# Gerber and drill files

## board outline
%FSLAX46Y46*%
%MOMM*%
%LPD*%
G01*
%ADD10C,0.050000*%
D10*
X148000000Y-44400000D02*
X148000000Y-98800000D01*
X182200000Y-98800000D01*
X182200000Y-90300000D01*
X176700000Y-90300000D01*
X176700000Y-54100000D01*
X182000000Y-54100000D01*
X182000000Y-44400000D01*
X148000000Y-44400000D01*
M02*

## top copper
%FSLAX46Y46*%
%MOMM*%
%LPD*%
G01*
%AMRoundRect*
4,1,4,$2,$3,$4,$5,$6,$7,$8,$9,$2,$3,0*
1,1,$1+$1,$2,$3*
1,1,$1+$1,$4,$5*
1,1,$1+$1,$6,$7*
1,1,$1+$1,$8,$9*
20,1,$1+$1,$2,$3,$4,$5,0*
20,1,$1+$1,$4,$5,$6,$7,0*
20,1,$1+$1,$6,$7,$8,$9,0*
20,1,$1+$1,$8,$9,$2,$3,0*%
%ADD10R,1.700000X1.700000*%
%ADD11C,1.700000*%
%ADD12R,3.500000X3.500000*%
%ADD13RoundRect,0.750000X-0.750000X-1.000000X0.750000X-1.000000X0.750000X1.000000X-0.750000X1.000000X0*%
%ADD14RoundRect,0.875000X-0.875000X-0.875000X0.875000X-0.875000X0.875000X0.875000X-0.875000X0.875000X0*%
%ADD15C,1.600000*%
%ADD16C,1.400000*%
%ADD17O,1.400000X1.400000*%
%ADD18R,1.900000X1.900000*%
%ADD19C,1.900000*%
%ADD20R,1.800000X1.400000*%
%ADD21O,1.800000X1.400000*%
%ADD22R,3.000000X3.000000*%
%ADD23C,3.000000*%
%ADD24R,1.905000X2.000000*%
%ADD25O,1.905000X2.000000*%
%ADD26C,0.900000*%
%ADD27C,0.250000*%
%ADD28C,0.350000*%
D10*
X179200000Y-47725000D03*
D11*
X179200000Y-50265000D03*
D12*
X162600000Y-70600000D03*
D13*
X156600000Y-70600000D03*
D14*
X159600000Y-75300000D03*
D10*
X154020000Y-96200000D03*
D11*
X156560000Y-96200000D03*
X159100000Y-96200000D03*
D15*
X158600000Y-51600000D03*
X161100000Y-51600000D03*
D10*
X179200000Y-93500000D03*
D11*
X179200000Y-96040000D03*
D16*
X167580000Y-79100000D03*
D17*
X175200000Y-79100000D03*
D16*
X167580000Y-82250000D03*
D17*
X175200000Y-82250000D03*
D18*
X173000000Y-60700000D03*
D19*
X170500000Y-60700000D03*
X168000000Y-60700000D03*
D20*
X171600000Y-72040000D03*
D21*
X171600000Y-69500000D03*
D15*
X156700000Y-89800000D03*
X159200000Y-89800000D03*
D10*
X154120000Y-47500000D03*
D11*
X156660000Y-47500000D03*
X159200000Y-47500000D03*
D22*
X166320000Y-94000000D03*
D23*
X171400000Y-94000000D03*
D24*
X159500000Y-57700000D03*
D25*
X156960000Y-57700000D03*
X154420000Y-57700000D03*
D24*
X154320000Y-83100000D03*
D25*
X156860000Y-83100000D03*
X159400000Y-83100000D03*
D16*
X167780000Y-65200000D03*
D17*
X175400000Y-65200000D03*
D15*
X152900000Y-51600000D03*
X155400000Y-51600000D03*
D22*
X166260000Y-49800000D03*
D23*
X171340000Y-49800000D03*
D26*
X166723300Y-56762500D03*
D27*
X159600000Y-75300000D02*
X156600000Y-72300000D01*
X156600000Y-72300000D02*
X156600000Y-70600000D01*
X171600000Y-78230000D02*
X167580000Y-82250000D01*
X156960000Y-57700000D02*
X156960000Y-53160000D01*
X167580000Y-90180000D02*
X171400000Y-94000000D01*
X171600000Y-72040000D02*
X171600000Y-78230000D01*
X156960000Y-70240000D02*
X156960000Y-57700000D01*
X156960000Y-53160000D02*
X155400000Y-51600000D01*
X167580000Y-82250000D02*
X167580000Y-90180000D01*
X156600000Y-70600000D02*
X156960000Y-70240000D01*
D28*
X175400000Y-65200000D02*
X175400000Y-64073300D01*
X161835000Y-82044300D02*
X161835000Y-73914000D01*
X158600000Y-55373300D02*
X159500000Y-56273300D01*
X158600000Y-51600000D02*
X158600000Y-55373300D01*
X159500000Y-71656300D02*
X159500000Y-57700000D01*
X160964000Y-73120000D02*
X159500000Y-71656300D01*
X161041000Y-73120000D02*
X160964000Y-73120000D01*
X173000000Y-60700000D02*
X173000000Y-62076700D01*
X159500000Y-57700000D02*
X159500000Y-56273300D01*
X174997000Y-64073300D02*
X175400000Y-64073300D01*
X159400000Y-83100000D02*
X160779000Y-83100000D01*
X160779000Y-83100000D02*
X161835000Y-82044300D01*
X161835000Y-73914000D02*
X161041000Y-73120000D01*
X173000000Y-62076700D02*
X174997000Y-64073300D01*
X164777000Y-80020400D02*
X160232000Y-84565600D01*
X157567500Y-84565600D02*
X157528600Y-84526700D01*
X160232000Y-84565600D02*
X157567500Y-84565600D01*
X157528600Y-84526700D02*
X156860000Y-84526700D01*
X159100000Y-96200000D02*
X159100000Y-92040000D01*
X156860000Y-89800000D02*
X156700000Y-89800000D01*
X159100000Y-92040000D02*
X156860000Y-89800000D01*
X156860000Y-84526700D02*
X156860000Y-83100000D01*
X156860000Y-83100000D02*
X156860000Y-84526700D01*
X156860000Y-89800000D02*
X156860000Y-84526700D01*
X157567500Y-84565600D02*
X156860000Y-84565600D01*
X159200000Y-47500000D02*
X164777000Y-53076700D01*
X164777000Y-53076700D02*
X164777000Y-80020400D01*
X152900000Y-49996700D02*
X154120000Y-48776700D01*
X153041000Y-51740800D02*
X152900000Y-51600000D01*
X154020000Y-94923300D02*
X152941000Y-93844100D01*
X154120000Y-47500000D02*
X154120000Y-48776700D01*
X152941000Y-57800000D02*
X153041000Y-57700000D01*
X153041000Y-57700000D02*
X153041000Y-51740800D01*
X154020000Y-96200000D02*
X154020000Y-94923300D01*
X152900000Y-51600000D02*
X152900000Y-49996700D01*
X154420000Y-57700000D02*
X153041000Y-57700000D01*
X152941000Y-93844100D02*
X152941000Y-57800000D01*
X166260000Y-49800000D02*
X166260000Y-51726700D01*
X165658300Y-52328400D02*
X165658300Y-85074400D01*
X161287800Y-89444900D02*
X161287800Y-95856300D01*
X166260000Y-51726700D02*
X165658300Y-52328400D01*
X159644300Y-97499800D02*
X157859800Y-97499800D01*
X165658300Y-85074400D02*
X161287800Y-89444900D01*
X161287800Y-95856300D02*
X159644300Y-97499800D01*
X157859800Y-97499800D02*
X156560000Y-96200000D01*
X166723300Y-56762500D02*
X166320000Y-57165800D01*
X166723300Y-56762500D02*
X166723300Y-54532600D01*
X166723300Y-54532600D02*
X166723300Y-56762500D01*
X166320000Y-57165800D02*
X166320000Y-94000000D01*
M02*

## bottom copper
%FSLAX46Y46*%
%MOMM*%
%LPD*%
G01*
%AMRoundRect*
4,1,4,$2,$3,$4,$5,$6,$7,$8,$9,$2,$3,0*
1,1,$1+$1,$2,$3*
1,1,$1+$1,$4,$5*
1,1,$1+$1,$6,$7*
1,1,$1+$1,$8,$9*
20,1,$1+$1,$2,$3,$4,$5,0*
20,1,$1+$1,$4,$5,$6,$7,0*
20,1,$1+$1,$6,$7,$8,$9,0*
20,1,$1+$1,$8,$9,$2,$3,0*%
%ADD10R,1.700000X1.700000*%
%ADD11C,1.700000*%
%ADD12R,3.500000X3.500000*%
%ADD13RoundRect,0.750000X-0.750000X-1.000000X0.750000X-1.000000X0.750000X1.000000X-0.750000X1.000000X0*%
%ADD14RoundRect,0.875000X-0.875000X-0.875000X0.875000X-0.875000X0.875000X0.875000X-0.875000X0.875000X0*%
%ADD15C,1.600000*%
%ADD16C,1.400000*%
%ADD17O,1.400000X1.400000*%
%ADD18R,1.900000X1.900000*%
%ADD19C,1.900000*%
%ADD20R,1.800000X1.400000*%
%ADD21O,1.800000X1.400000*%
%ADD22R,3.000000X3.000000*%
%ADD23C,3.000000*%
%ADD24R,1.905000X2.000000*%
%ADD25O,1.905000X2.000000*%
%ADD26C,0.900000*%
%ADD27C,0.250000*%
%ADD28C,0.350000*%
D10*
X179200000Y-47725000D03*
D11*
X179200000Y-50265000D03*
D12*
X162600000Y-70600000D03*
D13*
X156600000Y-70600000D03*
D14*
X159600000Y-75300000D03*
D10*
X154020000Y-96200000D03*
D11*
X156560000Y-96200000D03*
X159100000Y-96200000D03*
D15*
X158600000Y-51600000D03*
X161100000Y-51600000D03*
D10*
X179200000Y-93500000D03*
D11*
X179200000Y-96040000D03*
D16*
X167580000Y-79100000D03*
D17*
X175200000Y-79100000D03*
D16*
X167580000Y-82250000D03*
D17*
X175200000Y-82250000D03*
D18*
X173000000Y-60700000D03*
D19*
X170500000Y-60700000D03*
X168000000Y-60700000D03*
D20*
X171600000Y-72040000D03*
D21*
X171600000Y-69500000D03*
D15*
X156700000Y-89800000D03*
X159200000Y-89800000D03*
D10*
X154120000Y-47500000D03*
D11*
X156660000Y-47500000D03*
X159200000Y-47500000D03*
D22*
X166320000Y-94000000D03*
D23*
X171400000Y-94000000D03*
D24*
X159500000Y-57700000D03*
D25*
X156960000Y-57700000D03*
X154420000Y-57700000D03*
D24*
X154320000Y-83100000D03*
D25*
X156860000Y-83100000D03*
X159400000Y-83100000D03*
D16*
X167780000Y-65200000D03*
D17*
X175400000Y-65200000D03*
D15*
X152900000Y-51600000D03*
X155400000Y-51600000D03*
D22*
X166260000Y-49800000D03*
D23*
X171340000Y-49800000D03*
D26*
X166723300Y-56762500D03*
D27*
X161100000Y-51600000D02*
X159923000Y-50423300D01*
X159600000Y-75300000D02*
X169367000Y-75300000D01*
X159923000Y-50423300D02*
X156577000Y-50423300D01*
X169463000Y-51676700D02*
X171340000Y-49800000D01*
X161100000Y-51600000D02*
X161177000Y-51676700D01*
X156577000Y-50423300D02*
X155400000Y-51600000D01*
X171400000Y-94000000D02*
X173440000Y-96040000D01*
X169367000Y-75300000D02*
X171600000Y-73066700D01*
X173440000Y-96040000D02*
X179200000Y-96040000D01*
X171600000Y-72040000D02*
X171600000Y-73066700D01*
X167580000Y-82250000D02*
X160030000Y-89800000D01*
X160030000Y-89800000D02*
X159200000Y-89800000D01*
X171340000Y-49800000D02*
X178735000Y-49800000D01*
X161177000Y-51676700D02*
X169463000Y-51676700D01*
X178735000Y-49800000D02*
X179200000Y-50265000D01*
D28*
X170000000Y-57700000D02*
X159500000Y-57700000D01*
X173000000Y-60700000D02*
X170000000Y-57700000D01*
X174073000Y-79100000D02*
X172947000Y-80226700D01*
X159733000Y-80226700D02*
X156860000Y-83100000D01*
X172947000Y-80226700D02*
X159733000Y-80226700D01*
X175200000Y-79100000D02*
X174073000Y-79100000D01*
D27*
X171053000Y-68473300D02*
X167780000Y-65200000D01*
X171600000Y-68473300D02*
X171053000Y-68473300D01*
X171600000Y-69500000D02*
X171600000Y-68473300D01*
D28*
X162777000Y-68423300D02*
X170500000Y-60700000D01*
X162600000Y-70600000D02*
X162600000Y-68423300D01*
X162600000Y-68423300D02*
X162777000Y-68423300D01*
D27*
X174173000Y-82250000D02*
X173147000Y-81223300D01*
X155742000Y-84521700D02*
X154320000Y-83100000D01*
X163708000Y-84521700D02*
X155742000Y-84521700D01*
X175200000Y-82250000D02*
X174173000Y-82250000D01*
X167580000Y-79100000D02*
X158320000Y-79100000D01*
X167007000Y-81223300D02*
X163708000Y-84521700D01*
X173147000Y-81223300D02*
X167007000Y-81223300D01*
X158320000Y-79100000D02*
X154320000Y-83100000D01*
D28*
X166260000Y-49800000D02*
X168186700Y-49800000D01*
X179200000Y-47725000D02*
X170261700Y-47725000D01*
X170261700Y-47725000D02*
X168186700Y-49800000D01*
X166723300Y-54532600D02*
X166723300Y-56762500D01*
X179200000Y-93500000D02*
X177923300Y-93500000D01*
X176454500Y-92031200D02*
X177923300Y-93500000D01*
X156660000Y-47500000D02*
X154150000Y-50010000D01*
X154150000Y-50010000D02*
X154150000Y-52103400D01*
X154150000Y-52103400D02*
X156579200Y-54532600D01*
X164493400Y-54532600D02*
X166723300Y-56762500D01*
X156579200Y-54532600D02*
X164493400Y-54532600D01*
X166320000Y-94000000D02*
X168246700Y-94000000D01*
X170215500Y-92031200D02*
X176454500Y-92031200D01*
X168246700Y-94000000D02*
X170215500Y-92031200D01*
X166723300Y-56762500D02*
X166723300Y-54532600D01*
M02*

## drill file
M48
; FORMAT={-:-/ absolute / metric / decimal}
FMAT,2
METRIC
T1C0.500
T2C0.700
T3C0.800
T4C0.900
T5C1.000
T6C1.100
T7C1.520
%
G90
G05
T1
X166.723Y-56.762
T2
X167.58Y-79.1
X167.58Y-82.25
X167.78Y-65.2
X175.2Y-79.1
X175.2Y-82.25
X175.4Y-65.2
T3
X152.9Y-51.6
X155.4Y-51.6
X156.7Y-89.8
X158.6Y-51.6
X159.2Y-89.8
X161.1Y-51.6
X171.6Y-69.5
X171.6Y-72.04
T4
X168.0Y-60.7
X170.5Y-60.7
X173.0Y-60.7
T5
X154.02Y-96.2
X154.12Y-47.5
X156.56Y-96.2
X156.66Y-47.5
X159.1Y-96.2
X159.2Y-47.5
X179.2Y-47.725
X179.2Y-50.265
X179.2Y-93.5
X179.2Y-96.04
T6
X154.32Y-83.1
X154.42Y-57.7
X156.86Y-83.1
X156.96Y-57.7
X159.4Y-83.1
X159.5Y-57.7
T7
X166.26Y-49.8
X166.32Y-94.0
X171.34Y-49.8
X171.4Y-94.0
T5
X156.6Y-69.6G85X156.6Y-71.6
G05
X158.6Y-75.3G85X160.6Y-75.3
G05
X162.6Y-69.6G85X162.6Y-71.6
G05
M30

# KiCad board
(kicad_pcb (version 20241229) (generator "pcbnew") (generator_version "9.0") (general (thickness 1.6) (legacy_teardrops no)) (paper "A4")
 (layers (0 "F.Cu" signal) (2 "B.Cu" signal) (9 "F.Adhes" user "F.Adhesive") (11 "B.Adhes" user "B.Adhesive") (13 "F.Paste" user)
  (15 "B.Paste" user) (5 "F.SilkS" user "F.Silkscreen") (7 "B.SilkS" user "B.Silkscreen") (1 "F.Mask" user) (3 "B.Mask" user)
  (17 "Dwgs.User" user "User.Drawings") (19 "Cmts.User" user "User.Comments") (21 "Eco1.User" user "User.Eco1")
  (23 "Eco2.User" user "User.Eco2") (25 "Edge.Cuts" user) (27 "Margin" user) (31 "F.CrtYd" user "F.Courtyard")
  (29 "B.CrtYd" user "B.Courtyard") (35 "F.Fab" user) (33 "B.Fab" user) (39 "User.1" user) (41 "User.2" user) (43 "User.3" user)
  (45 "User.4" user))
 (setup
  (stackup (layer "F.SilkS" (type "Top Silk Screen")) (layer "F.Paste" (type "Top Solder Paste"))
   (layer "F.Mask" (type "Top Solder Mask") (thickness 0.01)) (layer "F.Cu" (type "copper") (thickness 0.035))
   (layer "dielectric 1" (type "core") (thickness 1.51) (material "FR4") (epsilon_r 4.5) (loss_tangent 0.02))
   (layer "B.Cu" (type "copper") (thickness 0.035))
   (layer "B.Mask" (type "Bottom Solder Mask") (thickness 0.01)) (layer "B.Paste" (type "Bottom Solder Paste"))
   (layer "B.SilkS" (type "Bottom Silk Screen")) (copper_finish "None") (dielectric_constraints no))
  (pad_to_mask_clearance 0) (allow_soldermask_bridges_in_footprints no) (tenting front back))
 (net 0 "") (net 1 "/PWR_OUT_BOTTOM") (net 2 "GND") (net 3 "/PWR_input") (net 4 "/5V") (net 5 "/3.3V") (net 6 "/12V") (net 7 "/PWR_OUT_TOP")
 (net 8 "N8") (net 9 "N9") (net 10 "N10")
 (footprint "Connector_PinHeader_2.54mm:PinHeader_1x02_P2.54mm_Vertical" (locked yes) (layer "F.Cu") (at 179.2 47.725)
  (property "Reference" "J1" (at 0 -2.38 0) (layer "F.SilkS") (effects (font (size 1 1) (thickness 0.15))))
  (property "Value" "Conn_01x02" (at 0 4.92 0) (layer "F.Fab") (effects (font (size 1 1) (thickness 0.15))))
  (pad "1" thru_hole rect (at 0 0) (size 1.7 1.7) (drill 1) (layers "*.Cu" "*.Mask") (remove_unused_layers no) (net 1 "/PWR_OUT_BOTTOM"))
  (pad "2" thru_hole circle (at 0 2.54) (size 1.7 1.7) (drill 1) (layers "*.Cu" "*.Mask") (remove_unused_layers no) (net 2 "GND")))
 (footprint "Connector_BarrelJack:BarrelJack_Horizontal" (layer "F.Cu") (at 162.6 70.6)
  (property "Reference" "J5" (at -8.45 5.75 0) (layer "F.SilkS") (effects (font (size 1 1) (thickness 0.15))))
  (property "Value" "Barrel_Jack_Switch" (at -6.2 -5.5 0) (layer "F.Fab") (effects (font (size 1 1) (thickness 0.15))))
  (pad "1" thru_hole rect (at 0 0) (size 3.5 3.5) (drill oval 1 3) (layers "*.Cu" "*.Mask") (remove_unused_layers no) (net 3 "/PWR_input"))
  (pad "2" thru_hole roundrect (at -6 0) (size 3 3.5) (drill oval 1 3) (layers "*.Cu" "*.Mask") (remove_unused_layers no)
   (roundrect_rratio 0.25) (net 2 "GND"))
  (pad "3" thru_hole roundrect (at -3 4.7) (size 3.5 3.5) (drill oval 3 1) (layers "*.Cu" "*.Mask") (remove_unused_layers no)
   (roundrect_rratio 0.25) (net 2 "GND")))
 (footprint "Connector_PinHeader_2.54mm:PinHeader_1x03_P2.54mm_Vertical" (layer "F.Cu") (at 154.02 96.2 90)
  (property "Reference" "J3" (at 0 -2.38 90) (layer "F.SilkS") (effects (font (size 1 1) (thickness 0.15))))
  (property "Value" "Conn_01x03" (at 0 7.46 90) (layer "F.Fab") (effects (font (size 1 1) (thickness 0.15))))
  (pad "1" thru_hole rect (at 0 0 90) (size 1.7 1.7) (drill 1) (layers "*.Cu" "*.Mask") (remove_unused_layers no) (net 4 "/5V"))
  (pad "2" thru_hole circle (at 0 2.54 90) (size 1.7 1.7) (drill 1) (layers "*.Cu" "*.Mask") (remove_unused_layers no)
   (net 1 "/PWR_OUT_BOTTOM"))
  (pad "3" thru_hole circle (at 0 5.08 90) (size 1.7 1.7) (drill 1) (layers "*.Cu" "*.Mask") (remove_unused_layers no) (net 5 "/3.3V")))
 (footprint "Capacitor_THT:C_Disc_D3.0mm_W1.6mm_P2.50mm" (layer "F.Cu") (at 158.6 51.6)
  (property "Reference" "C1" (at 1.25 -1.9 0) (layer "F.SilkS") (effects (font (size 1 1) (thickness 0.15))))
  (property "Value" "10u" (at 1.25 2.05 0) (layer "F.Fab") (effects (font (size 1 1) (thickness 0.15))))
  (pad "1" thru_hole circle (at 0 0) (size 1.6 1.6) (drill 0.8) (layers "*.Cu" "*.Mask") (remove_unused_layers no) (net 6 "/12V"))
  (pad "2" thru_hole circle (at 2.5 0) (size 1.6 1.6) (drill 0.8) (layers "*.Cu" "*.Mask") (remove_unused_layers no) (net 2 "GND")))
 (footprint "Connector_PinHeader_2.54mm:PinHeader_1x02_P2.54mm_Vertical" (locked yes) (layer "F.Cu") (at 179.2 93.5)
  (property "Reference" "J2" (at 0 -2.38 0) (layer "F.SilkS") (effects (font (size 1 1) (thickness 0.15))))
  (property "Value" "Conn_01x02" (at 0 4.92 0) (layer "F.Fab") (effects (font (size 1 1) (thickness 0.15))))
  (pad "1" thru_hole rect (at 0 0) (size 1.7 1.7) (drill 1) (layers "*.Cu" "*.Mask") (remove_unused_layers no) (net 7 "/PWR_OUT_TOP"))
  (pad "2" thru_hole circle (at 0 2.54) (size 1.7 1.7) (drill 1) (layers "*.Cu" "*.Mask") (remove_unused_layers no) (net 2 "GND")))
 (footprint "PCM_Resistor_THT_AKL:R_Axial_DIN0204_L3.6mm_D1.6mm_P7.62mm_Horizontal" (layer "F.Cu") (at 167.58 79.1)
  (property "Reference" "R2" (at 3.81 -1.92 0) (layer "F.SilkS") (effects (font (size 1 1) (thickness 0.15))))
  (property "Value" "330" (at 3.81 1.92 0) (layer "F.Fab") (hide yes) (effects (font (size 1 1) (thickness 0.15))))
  (pad "1" thru_hole circle (at 0 0) (size 1.4 1.4) (drill 0.7) (layers "*.Cu" "*.Mask") (remove_unused_layers no) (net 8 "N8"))
  (pad "2" thru_hole oval (at 7.62 0) (size 1.4 1.4) (drill 0.7) (layers "*.Cu" "*.Mask") (remove_unused_layers no) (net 5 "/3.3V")))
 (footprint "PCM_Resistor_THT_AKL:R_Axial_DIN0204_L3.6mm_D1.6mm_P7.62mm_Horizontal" (layer "F.Cu") (at 167.58 82.25)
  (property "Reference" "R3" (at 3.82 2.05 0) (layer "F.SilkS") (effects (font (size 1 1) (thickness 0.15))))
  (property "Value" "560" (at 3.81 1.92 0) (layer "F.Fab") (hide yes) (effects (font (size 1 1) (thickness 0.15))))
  (pad "1" thru_hole circle (at 0 0) (size 1.4 1.4) (drill 0.7) (layers "*.Cu" "*.Mask") (remove_unused_layers no) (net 2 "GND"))
  (pad "2" thru_hole oval (at 7.62 0) (size 1.4 1.4) (drill 0.7) (layers "*.Cu" "*.Mask") (remove_unused_layers no) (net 8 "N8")))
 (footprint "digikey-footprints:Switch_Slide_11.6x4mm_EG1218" (layer "F.Cu") (at 173 60.7 180)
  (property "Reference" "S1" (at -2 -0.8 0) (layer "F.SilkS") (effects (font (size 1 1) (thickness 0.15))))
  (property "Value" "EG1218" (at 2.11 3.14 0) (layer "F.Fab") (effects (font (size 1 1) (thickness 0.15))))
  (pad "1" thru_hole rect (at 0 0 180) (size 1.9 1.9) (drill 0.9) (layers "*.Cu" "*.Mask") (remove_unused_layers no) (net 6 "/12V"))
  (pad "2" thru_hole circle (at 2.5 0 180) (size 1.9 1.9) (drill 0.9) (layers "*.Cu" "*.Mask") (remove_unused_layers no)
   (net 3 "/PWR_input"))
  (pad "3" thru_hole circle (at 5 0 180) (size 1.9 1.9) (drill 0.9) (layers "*.Cu" "*.Mask") (remove_unused_layers no) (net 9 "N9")))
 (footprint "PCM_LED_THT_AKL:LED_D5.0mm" (layer "F.Cu") (at 171.6 72.04 90)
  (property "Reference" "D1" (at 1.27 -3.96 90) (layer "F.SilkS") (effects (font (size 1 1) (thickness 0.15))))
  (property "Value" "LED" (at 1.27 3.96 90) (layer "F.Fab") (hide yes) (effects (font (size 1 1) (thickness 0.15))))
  (pad "1" thru_hole rect (at 0 0 90) (size 1.4 1.8) (drill 0.8) (layers "*.Cu" "*.Mask") (remove_unused_layers no) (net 2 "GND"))
  (pad "2" thru_hole oval (at 2.54 0 90) (size 1.4 1.8) (drill 0.8) (layers "*.Cu" "*.Mask") (remove_unused_layers no) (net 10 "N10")))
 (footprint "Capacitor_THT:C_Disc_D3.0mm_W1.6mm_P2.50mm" (layer "F.Cu") (at 156.7 89.8)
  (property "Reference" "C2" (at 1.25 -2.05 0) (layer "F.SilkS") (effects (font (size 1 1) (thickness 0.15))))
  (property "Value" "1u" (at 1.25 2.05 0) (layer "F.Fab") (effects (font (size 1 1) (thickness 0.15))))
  (pad "1" thru_hole circle (at 0 0) (size 1.6 1.6) (drill 0.8) (layers "*.Cu" "*.Mask") (remove_unused_layers no) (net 5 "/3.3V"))
  (pad "2" thru_hole circle (at 2.5 0) (size 1.6 1.6) (drill 0.8) (layers "*.Cu" "*.Mask") (remove_unused_layers no) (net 2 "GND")))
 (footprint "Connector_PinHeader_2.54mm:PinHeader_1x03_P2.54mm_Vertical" (layer "F.Cu") (at 154.12 47.5 90)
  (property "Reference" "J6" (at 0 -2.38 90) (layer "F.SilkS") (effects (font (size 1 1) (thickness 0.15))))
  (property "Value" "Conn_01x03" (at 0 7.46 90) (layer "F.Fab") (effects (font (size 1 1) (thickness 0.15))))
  (pad "1" thru_hole rect (at 0 0 90) (size 1.7 1.7) (drill 1) (layers "*.Cu" "*.Mask") (remove_unused_layers no) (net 4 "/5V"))
  (pad "2" thru_hole circle (at 0 2.54 90) (size 1.7 1.7) (drill 1) (layers "*.Cu" "*.Mask") (remove_unused_layers no)
   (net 7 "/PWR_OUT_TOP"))
  (pad "3" thru_hole circle (at 0 5.08 90) (size 1.7 1.7) (drill 1) (layers "*.Cu" "*.Mask") (remove_unused_layers no) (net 5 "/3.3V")))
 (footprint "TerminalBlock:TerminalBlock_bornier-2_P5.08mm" (layer "F.Cu") (at 166.32 94)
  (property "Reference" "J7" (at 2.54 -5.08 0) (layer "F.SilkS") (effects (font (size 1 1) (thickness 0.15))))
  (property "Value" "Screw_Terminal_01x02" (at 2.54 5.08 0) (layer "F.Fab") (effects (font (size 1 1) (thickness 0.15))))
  (pad "1" thru_hole rect (at 0 0) (size 3 3) (drill 1.52) (layers "*.Cu" "*.Mask") (remove_unused_layers no) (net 7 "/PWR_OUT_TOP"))
  (pad "2" thru_hole circle (at 5.08 0) (size 3 3) (drill 1.52) (layers "*.Cu" "*.Mask") (remove_unused_layers no) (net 2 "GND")))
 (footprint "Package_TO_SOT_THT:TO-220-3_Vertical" (layer "F.Cu") (at 159.5 57.7 180)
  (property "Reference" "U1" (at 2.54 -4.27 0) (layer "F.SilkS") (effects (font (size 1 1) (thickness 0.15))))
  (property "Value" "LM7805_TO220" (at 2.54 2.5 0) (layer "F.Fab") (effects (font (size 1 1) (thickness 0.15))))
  (pad "1" thru_hole rect (at 0 0 180) (size 1.905 2) (drill 1.1) (layers "*.Cu" "*.Mask") (remove_unused_layers no) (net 6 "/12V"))
  (pad "2" thru_hole oval (at 2.54 0 180) (size 1.905 2) (drill 1.1) (layers "*.Cu" "*.Mask") (remove_unused_layers no) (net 2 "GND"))
  (pad "3" thru_hole oval (at 5.08 0 180) (size 1.905 2) (drill 1.1) (layers "*.Cu" "*.Mask") (remove_unused_layers no) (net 4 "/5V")))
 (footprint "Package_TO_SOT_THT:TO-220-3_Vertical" (layer "F.Cu") (at 154.32 83.1)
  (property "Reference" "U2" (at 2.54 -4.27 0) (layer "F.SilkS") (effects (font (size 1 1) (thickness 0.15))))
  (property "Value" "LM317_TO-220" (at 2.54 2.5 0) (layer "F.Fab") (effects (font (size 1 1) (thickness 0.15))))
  (pad "1" thru_hole rect (at 0 0) (size 1.905 2) (drill 1.1) (layers "*.Cu" "*.Mask") (remove_unused_layers no) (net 8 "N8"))
  (pad "2" thru_hole oval (at 2.54 0) (size 1.905 2) (drill 1.1) (layers "*.Cu" "*.Mask") (remove_unused_layers no) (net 5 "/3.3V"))
  (pad "3" thru_hole oval (at 5.08 0) (size 1.905 2) (drill 1.1) (layers "*.Cu" "*.Mask") (remove_unused_layers no) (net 6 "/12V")))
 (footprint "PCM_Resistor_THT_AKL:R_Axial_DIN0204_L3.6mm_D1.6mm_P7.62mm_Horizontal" (layer "F.Cu") (at 167.78 65.2)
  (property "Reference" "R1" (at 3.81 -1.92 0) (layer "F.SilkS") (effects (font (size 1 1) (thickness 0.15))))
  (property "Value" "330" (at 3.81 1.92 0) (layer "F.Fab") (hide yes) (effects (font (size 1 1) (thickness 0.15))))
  (pad "1" thru_hole circle (at 0 0) (size 1.4 1.4) (drill 0.7) (layers "*.Cu" "*.Mask") (remove_unused_layers no) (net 10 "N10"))
  (pad "2" thru_hole oval (at 7.62 0) (size 1.4 1.4) (drill 0.7) (layers "*.Cu" "*.Mask") (remove_unused_layers no) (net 6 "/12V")))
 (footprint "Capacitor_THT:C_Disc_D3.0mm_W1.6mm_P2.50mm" (layer "F.Cu") (at 152.9 51.6)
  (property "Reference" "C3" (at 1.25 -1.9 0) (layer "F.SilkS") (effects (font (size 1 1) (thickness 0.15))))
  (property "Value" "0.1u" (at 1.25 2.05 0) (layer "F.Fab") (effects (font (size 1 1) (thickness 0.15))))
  (pad "1" thru_hole circle (at 0 0) (size 1.6 1.6) (drill 0.8) (layers "*.Cu" "*.Mask") (remove_unused_layers no) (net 4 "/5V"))
  (pad "2" thru_hole circle (at 2.5 0) (size 1.6 1.6) (drill 0.8) (layers "*.Cu" "*.Mask") (remove_unused_layers no) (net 2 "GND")))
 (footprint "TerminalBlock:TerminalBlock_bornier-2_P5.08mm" (layer "F.Cu") (at 166.26 49.8)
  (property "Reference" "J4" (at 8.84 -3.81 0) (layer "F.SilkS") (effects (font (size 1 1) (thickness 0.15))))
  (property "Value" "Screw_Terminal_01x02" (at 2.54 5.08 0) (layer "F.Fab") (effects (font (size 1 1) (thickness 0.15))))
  (pad "1" thru_hole rect (at 0 0) (size 3 3) (drill 1.52) (layers "*.Cu" "*.Mask") (remove_unused_layers no) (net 1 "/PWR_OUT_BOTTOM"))
  (pad "2" thru_hole circle (at 5.08 0) (size 3 3) (drill 1.52) (layers "*.Cu" "*.Mask") (remove_unused_layers no) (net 2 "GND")))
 (gr_poly
  (pts (xy 148 44.4) (xy 148 98.8) (xy 182.2 98.8) (xy 182.2 90.3) (xy 176.7 90.3) (xy 176.7 54.1) (xy 182 54.1) (xy 182 44.4))
  (stroke (width 0.05) (type solid)) (fill no) (layer "Edge.Cuts"))
 (segment (start 159.6 75.3) (end 156.6 72.3) (width 0.25) (layer "F.Cu") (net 2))
 (segment (start 156.6 72.3) (end 156.6 70.6) (width 0.25) (layer "F.Cu") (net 2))
 (segment (start 171.6 78.23) (end 167.58 82.25) (width 0.25) (layer "F.Cu") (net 2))
 (segment (start 156.96 57.7) (end 156.96 53.16) (width 0.25) (layer "F.Cu") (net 2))
 (segment (start 167.58 90.18) (end 171.4 94) (width 0.25) (layer "F.Cu") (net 2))
 (segment (start 171.6 72.04) (end 171.6 78.23) (width 0.25) (layer "F.Cu") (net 2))
 (segment (start 156.96 70.24) (end 156.96 57.7) (width 0.25) (layer "F.Cu") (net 2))
 (segment (start 156.96 53.16) (end 155.4 51.6) (width 0.25) (layer "F.Cu") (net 2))
 (segment (start 167.58 82.25) (end 167.58 90.18) (width 0.25) (layer "F.Cu") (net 2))
 (segment (start 156.6 70.6) (end 156.96 70.24) (width 0.25) (layer "F.Cu") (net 2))
 (segment (start 161.1 51.6) (end 159.923 50.4233) (width 0.25) (layer "B.Cu") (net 2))
 (segment (start 159.6 75.3) (end 169.367 75.3) (width 0.25) (layer "B.Cu") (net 2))
 (segment (start 159.923 50.4233) (end 156.577 50.4233) (width 0.25) (layer "B.Cu") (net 2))
 (segment (start 169.463 51.6767) (end 171.34 49.8) (width 0.25) (layer "B.Cu") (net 2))
 (segment (start 161.1 51.6) (end 161.177 51.6767) (width 0.25) (layer "B.Cu") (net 2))
 (segment (start 156.577 50.4233) (end 155.4 51.6) (width 0.25) (layer "B.Cu") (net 2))
 (segment (start 171.4 94) (end 173.44 96.04) (width 0.25) (layer "B.Cu") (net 2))
 (segment (start 169.367 75.3) (end 171.6 73.0667) (width 0.25) (layer "B.Cu") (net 2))
 (segment (start 173.44 96.04) (end 179.2 96.04) (width 0.25) (layer "B.Cu") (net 2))
 (segment (start 171.6 72.04) (end 171.6 73.0667) (width 0.25) (layer "B.Cu") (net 2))
 (segment (start 167.58 82.25) (end 160.03 89.8) (width 0.25) (layer "B.Cu") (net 2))
 (segment (start 160.03 89.8) (end 159.2 89.8) (width 0.25) (layer "B.Cu") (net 2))
 (segment (start 171.34 49.8) (end 178.735 49.8) (width 0.25) (layer "B.Cu") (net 2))
 (segment (start 161.177 51.6767) (end 169.463 51.6767) (width 0.25) (layer "B.Cu") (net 2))
 (segment (start 178.735 49.8) (end 179.2 50.265) (width 0.25) (layer "B.Cu") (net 2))
 (segment (start 175.4 65.2) (end 175.4 64.0733) (width 0.35) (layer "F.Cu") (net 6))
 (segment (start 161.835 82.0443) (end 161.835 73.914) (width 0.35) (layer "F.Cu") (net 6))
 (segment (start 158.6 55.3733) (end 159.5 56.2733) (width 0.35) (layer "F.Cu") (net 6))
 (segment (start 158.6 51.6) (end 158.6 55.3733) (width 0.35) (layer "F.Cu") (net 6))
 (segment (start 159.5 71.6563) (end 159.5 57.7) (width 0.35) (layer "F.Cu") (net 6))
 (segment (start 160.964 73.12) (end 159.5 71.6563) (width 0.35) (layer "F.Cu") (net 6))
 (segment (start 161.041 73.12) (end 160.964 73.12) (width 0.35) (layer "F.Cu") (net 6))
 (segment (start 173 60.7) (end 173 62.0767) (width 0.35) (layer "F.Cu") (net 6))
 (segment (start 159.5 57.7) (end 159.5 56.2733) (width 0.35) (layer "F.Cu") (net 6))
 (segment (start 174.997 64.0733) (end 175.4 64.0733) (width 0.35) (layer "F.Cu") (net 6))
 (segment (start 159.4 83.1) (end 160.779 83.1) (width 0.35) (layer "F.Cu") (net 6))
 (segment (start 160.779 83.1) (end 161.835 82.0443) (width 0.35) (layer "F.Cu") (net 6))
 (segment (start 161.835 73.914) (end 161.041 73.12) (width 0.35) (layer "F.Cu") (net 6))
 (segment (start 173 62.0767) (end 174.997 64.0733) (width 0.35) (layer "F.Cu") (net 6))
 (segment (start 170 57.7) (end 159.5 57.7) (width 0.35) (layer "B.Cu") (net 6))
 (segment (start 173 60.7) (end 170 57.7) (width 0.35) (layer "B.Cu") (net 6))
 (segment (start 164.777 80.0204) (end 160.232 84.5656) (width 0.35) (layer "F.Cu") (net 5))
 (segment (start 157.5675 84.5656) (end 157.5286 84.5267) (width 0.35) (layer "F.Cu") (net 5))
 (segment (start 160.232 84.5656) (end 157.5675 84.5656) (width 0.35) (layer "F.Cu") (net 5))
 (segment (start 157.5286 84.5267) (end 156.86 84.5267) (width 0.35) (layer "F.Cu") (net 5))
 (segment (start 159.1 96.2) (end 159.1 92.04) (width 0.35) (layer "F.Cu") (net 5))
 (segment (start 156.86 89.8) (end 156.7 89.8) (width 0.35) (layer "F.Cu") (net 5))
 (segment (start 159.1 92.04) (end 156.86 89.8) (width 0.35) (layer "F.Cu") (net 5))
 (segment (start 156.86 84.5267) (end 156.86 83.1) (width 0.35) (layer "F.Cu") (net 5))
 (segment (start 156.86 83.1) (end 156.86 84.5267) (width 0.35) (layer "F.Cu") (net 5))
 (segment (start 156.86 89.8) (end 156.86 84.5267) (width 0.35) (layer "F.Cu") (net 5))
 (segment (start 157.5675 84.5656) (end 156.86 84.5656) (width 0.35) (layer "F.Cu") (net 5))
 (segment (start 159.2 47.5) (end 164.777 53.0767) (width 0.35) (layer "F.Cu") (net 5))
 (segment (start 164.777 53.0767) (end 164.777 80.0204) (width 0.35) (layer "F.Cu") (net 5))
 (segment (start 174.073 79.1) (end 172.947 80.2267) (width 0.35) (layer "B.Cu") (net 5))
 (segment (start 159.733 80.2267) (end 156.86 83.1) (width 0.35) (layer "B.Cu") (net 5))
 (segment (start 172.947 80.2267) (end 159.733 80.2267) (width 0.35) (layer "B.Cu") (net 5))
 (segment (start 175.2 79.1) (end 174.073 79.1) (width 0.35) (layer "B.Cu") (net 5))
 (segment (start 152.9 49.9967) (end 154.12 48.7767) (width 0.35) (layer "F.Cu") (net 4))
 (segment (start 153.041 51.7408) (end 152.9 51.6) (width 0.35) (layer "F.Cu") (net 4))
 (segment (start 154.02 94.9233) (end 152.941 93.8441) (width 0.35) (layer "F.Cu") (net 4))
 (segment (start 154.12 47.5) (end 154.12 48.7767) (width 0.35) (layer "F.Cu") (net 4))
 (segment (start 152.941 57.8) (end 153.041 57.7) (width 0.35) (layer "F.Cu") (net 4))
 (segment (start 153.041 57.7) (end 153.041 51.7408) (width 0.35) (layer "F.Cu") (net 4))
 (segment (start 154.02 96.2) (end 154.02 94.9233) (width 0.35) (layer "F.Cu") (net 4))
 (segment (start 152.9 51.6) (end 152.9 49.9967) (width 0.35) (layer "F.Cu") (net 4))
 (segment (start 154.42 57.7) (end 153.041 57.7) (width 0.35) (layer "F.Cu") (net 4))
 (segment (start 152.941 93.8441) (end 152.941 57.8) (width 0.35) (layer "F.Cu") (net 4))
 (segment (start 171.053 68.4733) (end 167.78 65.2) (width 0.25) (layer "B.Cu") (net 10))
 (segment (start 171.6 68.4733) (end 171.053 68.4733) (width 0.25) (layer "B.Cu") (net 10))
 (segment (start 171.6 69.5) (end 171.6 68.4733) (width 0.25) (layer "B.Cu") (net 10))
 (segment (start 162.777 68.4233) (end 170.5 60.7) (width 0.35) (layer "B.Cu") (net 3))
 (segment (start 162.6 70.6) (end 162.6 68.4233) (width 0.35) (layer "B.Cu") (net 3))
 (segment (start 162.6 68.4233) (end 162.777 68.4233) (width 0.35) (layer "B.Cu") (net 3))
 (segment (start 174.173 82.25) (end 173.147 81.2233) (width 0.25) (layer "B.Cu") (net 8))
 (segment (start 155.742 84.5217) (end 154.32 83.1) (width 0.25) (layer "B.Cu") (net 8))
 (segment (start 163.708 84.5217) (end 155.742 84.5217) (width 0.25) (layer "B.Cu") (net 8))
 (segment (start 175.2 82.25) (end 174.173 82.25) (width 0.25) (layer "B.Cu") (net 8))
 (segment (start 167.58 79.1) (end 158.32 79.1) (width 0.25) (layer "B.Cu") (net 8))
 (segment (start 167.007 81.2233) (end 163.708 84.5217) (width 0.25) (layer "B.Cu") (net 8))
 (segment (start 173.147 81.2233) (end 167.007 81.2233) (width 0.25) (layer "B.Cu") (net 8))
 (segment (start 158.32 79.1) (end 154.32 83.1) (width 0.25) (layer "B.Cu") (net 8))
 (segment (start 166.26 49.8) (end 166.26 51.7267) (width 0.35) (layer "F.Cu") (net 1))
 (segment (start 165.6583 52.3284) (end 165.6583 85.0744) (width 0.35) (layer "F.Cu") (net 1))
 (segment (start 161.2878 89.4449) (end 161.2878 95.8563) (width 0.35) (layer "F.Cu") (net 1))
 (segment (start 166.26 51.7267) (end 165.6583 52.3284) (width 0.35) (layer "F.Cu") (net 1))
 (segment (start 159.6443 97.4998) (end 157.8598 97.4998) (width 0.35) (layer "F.Cu") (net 1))
 (segment (start 165.6583 85.0744) (end 161.2878 89.4449) (width 0.35) (layer "F.Cu") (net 1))
 (segment (start 161.2878 95.8563) (end 159.6443 97.4998) (width 0.35) (layer "F.Cu") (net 1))
 (segment (start 157.8598 97.4998) (end 156.56 96.2) (width 0.35) (layer "F.Cu") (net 1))
 (segment (start 166.26 49.8) (end 168.1867 49.8) (width 0.35) (layer "B.Cu") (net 1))
 (segment (start 179.2 47.725) (end 170.2617 47.725) (width 0.35) (layer "B.Cu") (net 1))
 (segment (start 170.2617 47.725) (end 168.1867 49.8) (width 0.35) (layer "B.Cu") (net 1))
 (segment (start 166.7233 56.7625) (end 166.32 57.1658) (width 0.35) (layer "F.Cu") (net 7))
 (segment (start 166.7233 56.7625) (end 166.7233 54.5326) (width 0.35) (layer "F.Cu") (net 7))
 (segment (start 166.7233 54.5326) (end 166.7233 56.7625) (width 0.35) (layer "F.Cu") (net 7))
 (segment (start 166.32 57.1658) (end 166.32 94) (width 0.35) (layer "F.Cu") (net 7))
 (via (at 166.7233 56.7625) (size 0.9) (drill 0.5) (layers "F.Cu" "B.Cu") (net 7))
 (segment (start 166.7233 54.5326) (end 166.7233 56.7625) (width 0.35) (layer "B.Cu") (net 7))
 (segment (start 179.2 93.5) (end 177.9233 93.5) (width 0.35) (layer "B.Cu") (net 7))
 (segment (start 176.4545 92.0312) (end 177.9233 93.5) (width 0.35) (layer "B.Cu") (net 7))
 (segment (start 156.66 47.5) (end 154.15 50.01) (width 0.35) (layer "B.Cu") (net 7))
 (segment (start 154.15 50.01) (end 154.15 52.1034) (width 0.35) (layer "B.Cu") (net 7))
 (segment (start 154.15 52.1034) (end 156.5792 54.5326) (width 0.35) (layer "B.Cu") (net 7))
 (segment (start 164.4934 54.5326) (end 166.7233 56.7625) (width 0.35) (layer "B.Cu") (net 7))
 (segment (start 156.5792 54.5326) (end 164.4934 54.5326) (width 0.35) (layer "B.Cu") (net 7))
 (segment (start 166.32 94) (end 168.2467 94) (width 0.35) (layer "B.Cu") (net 7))
 (segment (start 170.2155 92.0312) (end 176.4545 92.0312) (width 0.35) (layer "B.Cu") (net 7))
 (segment (start 168.2467 94) (end 170.2155 92.0312) (width 0.35) (layer "B.Cu") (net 7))
 (segment (start 166.7233 56.7625) (end 166.7233 54.5326) (width 0.35) (layer "B.Cu") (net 7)))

